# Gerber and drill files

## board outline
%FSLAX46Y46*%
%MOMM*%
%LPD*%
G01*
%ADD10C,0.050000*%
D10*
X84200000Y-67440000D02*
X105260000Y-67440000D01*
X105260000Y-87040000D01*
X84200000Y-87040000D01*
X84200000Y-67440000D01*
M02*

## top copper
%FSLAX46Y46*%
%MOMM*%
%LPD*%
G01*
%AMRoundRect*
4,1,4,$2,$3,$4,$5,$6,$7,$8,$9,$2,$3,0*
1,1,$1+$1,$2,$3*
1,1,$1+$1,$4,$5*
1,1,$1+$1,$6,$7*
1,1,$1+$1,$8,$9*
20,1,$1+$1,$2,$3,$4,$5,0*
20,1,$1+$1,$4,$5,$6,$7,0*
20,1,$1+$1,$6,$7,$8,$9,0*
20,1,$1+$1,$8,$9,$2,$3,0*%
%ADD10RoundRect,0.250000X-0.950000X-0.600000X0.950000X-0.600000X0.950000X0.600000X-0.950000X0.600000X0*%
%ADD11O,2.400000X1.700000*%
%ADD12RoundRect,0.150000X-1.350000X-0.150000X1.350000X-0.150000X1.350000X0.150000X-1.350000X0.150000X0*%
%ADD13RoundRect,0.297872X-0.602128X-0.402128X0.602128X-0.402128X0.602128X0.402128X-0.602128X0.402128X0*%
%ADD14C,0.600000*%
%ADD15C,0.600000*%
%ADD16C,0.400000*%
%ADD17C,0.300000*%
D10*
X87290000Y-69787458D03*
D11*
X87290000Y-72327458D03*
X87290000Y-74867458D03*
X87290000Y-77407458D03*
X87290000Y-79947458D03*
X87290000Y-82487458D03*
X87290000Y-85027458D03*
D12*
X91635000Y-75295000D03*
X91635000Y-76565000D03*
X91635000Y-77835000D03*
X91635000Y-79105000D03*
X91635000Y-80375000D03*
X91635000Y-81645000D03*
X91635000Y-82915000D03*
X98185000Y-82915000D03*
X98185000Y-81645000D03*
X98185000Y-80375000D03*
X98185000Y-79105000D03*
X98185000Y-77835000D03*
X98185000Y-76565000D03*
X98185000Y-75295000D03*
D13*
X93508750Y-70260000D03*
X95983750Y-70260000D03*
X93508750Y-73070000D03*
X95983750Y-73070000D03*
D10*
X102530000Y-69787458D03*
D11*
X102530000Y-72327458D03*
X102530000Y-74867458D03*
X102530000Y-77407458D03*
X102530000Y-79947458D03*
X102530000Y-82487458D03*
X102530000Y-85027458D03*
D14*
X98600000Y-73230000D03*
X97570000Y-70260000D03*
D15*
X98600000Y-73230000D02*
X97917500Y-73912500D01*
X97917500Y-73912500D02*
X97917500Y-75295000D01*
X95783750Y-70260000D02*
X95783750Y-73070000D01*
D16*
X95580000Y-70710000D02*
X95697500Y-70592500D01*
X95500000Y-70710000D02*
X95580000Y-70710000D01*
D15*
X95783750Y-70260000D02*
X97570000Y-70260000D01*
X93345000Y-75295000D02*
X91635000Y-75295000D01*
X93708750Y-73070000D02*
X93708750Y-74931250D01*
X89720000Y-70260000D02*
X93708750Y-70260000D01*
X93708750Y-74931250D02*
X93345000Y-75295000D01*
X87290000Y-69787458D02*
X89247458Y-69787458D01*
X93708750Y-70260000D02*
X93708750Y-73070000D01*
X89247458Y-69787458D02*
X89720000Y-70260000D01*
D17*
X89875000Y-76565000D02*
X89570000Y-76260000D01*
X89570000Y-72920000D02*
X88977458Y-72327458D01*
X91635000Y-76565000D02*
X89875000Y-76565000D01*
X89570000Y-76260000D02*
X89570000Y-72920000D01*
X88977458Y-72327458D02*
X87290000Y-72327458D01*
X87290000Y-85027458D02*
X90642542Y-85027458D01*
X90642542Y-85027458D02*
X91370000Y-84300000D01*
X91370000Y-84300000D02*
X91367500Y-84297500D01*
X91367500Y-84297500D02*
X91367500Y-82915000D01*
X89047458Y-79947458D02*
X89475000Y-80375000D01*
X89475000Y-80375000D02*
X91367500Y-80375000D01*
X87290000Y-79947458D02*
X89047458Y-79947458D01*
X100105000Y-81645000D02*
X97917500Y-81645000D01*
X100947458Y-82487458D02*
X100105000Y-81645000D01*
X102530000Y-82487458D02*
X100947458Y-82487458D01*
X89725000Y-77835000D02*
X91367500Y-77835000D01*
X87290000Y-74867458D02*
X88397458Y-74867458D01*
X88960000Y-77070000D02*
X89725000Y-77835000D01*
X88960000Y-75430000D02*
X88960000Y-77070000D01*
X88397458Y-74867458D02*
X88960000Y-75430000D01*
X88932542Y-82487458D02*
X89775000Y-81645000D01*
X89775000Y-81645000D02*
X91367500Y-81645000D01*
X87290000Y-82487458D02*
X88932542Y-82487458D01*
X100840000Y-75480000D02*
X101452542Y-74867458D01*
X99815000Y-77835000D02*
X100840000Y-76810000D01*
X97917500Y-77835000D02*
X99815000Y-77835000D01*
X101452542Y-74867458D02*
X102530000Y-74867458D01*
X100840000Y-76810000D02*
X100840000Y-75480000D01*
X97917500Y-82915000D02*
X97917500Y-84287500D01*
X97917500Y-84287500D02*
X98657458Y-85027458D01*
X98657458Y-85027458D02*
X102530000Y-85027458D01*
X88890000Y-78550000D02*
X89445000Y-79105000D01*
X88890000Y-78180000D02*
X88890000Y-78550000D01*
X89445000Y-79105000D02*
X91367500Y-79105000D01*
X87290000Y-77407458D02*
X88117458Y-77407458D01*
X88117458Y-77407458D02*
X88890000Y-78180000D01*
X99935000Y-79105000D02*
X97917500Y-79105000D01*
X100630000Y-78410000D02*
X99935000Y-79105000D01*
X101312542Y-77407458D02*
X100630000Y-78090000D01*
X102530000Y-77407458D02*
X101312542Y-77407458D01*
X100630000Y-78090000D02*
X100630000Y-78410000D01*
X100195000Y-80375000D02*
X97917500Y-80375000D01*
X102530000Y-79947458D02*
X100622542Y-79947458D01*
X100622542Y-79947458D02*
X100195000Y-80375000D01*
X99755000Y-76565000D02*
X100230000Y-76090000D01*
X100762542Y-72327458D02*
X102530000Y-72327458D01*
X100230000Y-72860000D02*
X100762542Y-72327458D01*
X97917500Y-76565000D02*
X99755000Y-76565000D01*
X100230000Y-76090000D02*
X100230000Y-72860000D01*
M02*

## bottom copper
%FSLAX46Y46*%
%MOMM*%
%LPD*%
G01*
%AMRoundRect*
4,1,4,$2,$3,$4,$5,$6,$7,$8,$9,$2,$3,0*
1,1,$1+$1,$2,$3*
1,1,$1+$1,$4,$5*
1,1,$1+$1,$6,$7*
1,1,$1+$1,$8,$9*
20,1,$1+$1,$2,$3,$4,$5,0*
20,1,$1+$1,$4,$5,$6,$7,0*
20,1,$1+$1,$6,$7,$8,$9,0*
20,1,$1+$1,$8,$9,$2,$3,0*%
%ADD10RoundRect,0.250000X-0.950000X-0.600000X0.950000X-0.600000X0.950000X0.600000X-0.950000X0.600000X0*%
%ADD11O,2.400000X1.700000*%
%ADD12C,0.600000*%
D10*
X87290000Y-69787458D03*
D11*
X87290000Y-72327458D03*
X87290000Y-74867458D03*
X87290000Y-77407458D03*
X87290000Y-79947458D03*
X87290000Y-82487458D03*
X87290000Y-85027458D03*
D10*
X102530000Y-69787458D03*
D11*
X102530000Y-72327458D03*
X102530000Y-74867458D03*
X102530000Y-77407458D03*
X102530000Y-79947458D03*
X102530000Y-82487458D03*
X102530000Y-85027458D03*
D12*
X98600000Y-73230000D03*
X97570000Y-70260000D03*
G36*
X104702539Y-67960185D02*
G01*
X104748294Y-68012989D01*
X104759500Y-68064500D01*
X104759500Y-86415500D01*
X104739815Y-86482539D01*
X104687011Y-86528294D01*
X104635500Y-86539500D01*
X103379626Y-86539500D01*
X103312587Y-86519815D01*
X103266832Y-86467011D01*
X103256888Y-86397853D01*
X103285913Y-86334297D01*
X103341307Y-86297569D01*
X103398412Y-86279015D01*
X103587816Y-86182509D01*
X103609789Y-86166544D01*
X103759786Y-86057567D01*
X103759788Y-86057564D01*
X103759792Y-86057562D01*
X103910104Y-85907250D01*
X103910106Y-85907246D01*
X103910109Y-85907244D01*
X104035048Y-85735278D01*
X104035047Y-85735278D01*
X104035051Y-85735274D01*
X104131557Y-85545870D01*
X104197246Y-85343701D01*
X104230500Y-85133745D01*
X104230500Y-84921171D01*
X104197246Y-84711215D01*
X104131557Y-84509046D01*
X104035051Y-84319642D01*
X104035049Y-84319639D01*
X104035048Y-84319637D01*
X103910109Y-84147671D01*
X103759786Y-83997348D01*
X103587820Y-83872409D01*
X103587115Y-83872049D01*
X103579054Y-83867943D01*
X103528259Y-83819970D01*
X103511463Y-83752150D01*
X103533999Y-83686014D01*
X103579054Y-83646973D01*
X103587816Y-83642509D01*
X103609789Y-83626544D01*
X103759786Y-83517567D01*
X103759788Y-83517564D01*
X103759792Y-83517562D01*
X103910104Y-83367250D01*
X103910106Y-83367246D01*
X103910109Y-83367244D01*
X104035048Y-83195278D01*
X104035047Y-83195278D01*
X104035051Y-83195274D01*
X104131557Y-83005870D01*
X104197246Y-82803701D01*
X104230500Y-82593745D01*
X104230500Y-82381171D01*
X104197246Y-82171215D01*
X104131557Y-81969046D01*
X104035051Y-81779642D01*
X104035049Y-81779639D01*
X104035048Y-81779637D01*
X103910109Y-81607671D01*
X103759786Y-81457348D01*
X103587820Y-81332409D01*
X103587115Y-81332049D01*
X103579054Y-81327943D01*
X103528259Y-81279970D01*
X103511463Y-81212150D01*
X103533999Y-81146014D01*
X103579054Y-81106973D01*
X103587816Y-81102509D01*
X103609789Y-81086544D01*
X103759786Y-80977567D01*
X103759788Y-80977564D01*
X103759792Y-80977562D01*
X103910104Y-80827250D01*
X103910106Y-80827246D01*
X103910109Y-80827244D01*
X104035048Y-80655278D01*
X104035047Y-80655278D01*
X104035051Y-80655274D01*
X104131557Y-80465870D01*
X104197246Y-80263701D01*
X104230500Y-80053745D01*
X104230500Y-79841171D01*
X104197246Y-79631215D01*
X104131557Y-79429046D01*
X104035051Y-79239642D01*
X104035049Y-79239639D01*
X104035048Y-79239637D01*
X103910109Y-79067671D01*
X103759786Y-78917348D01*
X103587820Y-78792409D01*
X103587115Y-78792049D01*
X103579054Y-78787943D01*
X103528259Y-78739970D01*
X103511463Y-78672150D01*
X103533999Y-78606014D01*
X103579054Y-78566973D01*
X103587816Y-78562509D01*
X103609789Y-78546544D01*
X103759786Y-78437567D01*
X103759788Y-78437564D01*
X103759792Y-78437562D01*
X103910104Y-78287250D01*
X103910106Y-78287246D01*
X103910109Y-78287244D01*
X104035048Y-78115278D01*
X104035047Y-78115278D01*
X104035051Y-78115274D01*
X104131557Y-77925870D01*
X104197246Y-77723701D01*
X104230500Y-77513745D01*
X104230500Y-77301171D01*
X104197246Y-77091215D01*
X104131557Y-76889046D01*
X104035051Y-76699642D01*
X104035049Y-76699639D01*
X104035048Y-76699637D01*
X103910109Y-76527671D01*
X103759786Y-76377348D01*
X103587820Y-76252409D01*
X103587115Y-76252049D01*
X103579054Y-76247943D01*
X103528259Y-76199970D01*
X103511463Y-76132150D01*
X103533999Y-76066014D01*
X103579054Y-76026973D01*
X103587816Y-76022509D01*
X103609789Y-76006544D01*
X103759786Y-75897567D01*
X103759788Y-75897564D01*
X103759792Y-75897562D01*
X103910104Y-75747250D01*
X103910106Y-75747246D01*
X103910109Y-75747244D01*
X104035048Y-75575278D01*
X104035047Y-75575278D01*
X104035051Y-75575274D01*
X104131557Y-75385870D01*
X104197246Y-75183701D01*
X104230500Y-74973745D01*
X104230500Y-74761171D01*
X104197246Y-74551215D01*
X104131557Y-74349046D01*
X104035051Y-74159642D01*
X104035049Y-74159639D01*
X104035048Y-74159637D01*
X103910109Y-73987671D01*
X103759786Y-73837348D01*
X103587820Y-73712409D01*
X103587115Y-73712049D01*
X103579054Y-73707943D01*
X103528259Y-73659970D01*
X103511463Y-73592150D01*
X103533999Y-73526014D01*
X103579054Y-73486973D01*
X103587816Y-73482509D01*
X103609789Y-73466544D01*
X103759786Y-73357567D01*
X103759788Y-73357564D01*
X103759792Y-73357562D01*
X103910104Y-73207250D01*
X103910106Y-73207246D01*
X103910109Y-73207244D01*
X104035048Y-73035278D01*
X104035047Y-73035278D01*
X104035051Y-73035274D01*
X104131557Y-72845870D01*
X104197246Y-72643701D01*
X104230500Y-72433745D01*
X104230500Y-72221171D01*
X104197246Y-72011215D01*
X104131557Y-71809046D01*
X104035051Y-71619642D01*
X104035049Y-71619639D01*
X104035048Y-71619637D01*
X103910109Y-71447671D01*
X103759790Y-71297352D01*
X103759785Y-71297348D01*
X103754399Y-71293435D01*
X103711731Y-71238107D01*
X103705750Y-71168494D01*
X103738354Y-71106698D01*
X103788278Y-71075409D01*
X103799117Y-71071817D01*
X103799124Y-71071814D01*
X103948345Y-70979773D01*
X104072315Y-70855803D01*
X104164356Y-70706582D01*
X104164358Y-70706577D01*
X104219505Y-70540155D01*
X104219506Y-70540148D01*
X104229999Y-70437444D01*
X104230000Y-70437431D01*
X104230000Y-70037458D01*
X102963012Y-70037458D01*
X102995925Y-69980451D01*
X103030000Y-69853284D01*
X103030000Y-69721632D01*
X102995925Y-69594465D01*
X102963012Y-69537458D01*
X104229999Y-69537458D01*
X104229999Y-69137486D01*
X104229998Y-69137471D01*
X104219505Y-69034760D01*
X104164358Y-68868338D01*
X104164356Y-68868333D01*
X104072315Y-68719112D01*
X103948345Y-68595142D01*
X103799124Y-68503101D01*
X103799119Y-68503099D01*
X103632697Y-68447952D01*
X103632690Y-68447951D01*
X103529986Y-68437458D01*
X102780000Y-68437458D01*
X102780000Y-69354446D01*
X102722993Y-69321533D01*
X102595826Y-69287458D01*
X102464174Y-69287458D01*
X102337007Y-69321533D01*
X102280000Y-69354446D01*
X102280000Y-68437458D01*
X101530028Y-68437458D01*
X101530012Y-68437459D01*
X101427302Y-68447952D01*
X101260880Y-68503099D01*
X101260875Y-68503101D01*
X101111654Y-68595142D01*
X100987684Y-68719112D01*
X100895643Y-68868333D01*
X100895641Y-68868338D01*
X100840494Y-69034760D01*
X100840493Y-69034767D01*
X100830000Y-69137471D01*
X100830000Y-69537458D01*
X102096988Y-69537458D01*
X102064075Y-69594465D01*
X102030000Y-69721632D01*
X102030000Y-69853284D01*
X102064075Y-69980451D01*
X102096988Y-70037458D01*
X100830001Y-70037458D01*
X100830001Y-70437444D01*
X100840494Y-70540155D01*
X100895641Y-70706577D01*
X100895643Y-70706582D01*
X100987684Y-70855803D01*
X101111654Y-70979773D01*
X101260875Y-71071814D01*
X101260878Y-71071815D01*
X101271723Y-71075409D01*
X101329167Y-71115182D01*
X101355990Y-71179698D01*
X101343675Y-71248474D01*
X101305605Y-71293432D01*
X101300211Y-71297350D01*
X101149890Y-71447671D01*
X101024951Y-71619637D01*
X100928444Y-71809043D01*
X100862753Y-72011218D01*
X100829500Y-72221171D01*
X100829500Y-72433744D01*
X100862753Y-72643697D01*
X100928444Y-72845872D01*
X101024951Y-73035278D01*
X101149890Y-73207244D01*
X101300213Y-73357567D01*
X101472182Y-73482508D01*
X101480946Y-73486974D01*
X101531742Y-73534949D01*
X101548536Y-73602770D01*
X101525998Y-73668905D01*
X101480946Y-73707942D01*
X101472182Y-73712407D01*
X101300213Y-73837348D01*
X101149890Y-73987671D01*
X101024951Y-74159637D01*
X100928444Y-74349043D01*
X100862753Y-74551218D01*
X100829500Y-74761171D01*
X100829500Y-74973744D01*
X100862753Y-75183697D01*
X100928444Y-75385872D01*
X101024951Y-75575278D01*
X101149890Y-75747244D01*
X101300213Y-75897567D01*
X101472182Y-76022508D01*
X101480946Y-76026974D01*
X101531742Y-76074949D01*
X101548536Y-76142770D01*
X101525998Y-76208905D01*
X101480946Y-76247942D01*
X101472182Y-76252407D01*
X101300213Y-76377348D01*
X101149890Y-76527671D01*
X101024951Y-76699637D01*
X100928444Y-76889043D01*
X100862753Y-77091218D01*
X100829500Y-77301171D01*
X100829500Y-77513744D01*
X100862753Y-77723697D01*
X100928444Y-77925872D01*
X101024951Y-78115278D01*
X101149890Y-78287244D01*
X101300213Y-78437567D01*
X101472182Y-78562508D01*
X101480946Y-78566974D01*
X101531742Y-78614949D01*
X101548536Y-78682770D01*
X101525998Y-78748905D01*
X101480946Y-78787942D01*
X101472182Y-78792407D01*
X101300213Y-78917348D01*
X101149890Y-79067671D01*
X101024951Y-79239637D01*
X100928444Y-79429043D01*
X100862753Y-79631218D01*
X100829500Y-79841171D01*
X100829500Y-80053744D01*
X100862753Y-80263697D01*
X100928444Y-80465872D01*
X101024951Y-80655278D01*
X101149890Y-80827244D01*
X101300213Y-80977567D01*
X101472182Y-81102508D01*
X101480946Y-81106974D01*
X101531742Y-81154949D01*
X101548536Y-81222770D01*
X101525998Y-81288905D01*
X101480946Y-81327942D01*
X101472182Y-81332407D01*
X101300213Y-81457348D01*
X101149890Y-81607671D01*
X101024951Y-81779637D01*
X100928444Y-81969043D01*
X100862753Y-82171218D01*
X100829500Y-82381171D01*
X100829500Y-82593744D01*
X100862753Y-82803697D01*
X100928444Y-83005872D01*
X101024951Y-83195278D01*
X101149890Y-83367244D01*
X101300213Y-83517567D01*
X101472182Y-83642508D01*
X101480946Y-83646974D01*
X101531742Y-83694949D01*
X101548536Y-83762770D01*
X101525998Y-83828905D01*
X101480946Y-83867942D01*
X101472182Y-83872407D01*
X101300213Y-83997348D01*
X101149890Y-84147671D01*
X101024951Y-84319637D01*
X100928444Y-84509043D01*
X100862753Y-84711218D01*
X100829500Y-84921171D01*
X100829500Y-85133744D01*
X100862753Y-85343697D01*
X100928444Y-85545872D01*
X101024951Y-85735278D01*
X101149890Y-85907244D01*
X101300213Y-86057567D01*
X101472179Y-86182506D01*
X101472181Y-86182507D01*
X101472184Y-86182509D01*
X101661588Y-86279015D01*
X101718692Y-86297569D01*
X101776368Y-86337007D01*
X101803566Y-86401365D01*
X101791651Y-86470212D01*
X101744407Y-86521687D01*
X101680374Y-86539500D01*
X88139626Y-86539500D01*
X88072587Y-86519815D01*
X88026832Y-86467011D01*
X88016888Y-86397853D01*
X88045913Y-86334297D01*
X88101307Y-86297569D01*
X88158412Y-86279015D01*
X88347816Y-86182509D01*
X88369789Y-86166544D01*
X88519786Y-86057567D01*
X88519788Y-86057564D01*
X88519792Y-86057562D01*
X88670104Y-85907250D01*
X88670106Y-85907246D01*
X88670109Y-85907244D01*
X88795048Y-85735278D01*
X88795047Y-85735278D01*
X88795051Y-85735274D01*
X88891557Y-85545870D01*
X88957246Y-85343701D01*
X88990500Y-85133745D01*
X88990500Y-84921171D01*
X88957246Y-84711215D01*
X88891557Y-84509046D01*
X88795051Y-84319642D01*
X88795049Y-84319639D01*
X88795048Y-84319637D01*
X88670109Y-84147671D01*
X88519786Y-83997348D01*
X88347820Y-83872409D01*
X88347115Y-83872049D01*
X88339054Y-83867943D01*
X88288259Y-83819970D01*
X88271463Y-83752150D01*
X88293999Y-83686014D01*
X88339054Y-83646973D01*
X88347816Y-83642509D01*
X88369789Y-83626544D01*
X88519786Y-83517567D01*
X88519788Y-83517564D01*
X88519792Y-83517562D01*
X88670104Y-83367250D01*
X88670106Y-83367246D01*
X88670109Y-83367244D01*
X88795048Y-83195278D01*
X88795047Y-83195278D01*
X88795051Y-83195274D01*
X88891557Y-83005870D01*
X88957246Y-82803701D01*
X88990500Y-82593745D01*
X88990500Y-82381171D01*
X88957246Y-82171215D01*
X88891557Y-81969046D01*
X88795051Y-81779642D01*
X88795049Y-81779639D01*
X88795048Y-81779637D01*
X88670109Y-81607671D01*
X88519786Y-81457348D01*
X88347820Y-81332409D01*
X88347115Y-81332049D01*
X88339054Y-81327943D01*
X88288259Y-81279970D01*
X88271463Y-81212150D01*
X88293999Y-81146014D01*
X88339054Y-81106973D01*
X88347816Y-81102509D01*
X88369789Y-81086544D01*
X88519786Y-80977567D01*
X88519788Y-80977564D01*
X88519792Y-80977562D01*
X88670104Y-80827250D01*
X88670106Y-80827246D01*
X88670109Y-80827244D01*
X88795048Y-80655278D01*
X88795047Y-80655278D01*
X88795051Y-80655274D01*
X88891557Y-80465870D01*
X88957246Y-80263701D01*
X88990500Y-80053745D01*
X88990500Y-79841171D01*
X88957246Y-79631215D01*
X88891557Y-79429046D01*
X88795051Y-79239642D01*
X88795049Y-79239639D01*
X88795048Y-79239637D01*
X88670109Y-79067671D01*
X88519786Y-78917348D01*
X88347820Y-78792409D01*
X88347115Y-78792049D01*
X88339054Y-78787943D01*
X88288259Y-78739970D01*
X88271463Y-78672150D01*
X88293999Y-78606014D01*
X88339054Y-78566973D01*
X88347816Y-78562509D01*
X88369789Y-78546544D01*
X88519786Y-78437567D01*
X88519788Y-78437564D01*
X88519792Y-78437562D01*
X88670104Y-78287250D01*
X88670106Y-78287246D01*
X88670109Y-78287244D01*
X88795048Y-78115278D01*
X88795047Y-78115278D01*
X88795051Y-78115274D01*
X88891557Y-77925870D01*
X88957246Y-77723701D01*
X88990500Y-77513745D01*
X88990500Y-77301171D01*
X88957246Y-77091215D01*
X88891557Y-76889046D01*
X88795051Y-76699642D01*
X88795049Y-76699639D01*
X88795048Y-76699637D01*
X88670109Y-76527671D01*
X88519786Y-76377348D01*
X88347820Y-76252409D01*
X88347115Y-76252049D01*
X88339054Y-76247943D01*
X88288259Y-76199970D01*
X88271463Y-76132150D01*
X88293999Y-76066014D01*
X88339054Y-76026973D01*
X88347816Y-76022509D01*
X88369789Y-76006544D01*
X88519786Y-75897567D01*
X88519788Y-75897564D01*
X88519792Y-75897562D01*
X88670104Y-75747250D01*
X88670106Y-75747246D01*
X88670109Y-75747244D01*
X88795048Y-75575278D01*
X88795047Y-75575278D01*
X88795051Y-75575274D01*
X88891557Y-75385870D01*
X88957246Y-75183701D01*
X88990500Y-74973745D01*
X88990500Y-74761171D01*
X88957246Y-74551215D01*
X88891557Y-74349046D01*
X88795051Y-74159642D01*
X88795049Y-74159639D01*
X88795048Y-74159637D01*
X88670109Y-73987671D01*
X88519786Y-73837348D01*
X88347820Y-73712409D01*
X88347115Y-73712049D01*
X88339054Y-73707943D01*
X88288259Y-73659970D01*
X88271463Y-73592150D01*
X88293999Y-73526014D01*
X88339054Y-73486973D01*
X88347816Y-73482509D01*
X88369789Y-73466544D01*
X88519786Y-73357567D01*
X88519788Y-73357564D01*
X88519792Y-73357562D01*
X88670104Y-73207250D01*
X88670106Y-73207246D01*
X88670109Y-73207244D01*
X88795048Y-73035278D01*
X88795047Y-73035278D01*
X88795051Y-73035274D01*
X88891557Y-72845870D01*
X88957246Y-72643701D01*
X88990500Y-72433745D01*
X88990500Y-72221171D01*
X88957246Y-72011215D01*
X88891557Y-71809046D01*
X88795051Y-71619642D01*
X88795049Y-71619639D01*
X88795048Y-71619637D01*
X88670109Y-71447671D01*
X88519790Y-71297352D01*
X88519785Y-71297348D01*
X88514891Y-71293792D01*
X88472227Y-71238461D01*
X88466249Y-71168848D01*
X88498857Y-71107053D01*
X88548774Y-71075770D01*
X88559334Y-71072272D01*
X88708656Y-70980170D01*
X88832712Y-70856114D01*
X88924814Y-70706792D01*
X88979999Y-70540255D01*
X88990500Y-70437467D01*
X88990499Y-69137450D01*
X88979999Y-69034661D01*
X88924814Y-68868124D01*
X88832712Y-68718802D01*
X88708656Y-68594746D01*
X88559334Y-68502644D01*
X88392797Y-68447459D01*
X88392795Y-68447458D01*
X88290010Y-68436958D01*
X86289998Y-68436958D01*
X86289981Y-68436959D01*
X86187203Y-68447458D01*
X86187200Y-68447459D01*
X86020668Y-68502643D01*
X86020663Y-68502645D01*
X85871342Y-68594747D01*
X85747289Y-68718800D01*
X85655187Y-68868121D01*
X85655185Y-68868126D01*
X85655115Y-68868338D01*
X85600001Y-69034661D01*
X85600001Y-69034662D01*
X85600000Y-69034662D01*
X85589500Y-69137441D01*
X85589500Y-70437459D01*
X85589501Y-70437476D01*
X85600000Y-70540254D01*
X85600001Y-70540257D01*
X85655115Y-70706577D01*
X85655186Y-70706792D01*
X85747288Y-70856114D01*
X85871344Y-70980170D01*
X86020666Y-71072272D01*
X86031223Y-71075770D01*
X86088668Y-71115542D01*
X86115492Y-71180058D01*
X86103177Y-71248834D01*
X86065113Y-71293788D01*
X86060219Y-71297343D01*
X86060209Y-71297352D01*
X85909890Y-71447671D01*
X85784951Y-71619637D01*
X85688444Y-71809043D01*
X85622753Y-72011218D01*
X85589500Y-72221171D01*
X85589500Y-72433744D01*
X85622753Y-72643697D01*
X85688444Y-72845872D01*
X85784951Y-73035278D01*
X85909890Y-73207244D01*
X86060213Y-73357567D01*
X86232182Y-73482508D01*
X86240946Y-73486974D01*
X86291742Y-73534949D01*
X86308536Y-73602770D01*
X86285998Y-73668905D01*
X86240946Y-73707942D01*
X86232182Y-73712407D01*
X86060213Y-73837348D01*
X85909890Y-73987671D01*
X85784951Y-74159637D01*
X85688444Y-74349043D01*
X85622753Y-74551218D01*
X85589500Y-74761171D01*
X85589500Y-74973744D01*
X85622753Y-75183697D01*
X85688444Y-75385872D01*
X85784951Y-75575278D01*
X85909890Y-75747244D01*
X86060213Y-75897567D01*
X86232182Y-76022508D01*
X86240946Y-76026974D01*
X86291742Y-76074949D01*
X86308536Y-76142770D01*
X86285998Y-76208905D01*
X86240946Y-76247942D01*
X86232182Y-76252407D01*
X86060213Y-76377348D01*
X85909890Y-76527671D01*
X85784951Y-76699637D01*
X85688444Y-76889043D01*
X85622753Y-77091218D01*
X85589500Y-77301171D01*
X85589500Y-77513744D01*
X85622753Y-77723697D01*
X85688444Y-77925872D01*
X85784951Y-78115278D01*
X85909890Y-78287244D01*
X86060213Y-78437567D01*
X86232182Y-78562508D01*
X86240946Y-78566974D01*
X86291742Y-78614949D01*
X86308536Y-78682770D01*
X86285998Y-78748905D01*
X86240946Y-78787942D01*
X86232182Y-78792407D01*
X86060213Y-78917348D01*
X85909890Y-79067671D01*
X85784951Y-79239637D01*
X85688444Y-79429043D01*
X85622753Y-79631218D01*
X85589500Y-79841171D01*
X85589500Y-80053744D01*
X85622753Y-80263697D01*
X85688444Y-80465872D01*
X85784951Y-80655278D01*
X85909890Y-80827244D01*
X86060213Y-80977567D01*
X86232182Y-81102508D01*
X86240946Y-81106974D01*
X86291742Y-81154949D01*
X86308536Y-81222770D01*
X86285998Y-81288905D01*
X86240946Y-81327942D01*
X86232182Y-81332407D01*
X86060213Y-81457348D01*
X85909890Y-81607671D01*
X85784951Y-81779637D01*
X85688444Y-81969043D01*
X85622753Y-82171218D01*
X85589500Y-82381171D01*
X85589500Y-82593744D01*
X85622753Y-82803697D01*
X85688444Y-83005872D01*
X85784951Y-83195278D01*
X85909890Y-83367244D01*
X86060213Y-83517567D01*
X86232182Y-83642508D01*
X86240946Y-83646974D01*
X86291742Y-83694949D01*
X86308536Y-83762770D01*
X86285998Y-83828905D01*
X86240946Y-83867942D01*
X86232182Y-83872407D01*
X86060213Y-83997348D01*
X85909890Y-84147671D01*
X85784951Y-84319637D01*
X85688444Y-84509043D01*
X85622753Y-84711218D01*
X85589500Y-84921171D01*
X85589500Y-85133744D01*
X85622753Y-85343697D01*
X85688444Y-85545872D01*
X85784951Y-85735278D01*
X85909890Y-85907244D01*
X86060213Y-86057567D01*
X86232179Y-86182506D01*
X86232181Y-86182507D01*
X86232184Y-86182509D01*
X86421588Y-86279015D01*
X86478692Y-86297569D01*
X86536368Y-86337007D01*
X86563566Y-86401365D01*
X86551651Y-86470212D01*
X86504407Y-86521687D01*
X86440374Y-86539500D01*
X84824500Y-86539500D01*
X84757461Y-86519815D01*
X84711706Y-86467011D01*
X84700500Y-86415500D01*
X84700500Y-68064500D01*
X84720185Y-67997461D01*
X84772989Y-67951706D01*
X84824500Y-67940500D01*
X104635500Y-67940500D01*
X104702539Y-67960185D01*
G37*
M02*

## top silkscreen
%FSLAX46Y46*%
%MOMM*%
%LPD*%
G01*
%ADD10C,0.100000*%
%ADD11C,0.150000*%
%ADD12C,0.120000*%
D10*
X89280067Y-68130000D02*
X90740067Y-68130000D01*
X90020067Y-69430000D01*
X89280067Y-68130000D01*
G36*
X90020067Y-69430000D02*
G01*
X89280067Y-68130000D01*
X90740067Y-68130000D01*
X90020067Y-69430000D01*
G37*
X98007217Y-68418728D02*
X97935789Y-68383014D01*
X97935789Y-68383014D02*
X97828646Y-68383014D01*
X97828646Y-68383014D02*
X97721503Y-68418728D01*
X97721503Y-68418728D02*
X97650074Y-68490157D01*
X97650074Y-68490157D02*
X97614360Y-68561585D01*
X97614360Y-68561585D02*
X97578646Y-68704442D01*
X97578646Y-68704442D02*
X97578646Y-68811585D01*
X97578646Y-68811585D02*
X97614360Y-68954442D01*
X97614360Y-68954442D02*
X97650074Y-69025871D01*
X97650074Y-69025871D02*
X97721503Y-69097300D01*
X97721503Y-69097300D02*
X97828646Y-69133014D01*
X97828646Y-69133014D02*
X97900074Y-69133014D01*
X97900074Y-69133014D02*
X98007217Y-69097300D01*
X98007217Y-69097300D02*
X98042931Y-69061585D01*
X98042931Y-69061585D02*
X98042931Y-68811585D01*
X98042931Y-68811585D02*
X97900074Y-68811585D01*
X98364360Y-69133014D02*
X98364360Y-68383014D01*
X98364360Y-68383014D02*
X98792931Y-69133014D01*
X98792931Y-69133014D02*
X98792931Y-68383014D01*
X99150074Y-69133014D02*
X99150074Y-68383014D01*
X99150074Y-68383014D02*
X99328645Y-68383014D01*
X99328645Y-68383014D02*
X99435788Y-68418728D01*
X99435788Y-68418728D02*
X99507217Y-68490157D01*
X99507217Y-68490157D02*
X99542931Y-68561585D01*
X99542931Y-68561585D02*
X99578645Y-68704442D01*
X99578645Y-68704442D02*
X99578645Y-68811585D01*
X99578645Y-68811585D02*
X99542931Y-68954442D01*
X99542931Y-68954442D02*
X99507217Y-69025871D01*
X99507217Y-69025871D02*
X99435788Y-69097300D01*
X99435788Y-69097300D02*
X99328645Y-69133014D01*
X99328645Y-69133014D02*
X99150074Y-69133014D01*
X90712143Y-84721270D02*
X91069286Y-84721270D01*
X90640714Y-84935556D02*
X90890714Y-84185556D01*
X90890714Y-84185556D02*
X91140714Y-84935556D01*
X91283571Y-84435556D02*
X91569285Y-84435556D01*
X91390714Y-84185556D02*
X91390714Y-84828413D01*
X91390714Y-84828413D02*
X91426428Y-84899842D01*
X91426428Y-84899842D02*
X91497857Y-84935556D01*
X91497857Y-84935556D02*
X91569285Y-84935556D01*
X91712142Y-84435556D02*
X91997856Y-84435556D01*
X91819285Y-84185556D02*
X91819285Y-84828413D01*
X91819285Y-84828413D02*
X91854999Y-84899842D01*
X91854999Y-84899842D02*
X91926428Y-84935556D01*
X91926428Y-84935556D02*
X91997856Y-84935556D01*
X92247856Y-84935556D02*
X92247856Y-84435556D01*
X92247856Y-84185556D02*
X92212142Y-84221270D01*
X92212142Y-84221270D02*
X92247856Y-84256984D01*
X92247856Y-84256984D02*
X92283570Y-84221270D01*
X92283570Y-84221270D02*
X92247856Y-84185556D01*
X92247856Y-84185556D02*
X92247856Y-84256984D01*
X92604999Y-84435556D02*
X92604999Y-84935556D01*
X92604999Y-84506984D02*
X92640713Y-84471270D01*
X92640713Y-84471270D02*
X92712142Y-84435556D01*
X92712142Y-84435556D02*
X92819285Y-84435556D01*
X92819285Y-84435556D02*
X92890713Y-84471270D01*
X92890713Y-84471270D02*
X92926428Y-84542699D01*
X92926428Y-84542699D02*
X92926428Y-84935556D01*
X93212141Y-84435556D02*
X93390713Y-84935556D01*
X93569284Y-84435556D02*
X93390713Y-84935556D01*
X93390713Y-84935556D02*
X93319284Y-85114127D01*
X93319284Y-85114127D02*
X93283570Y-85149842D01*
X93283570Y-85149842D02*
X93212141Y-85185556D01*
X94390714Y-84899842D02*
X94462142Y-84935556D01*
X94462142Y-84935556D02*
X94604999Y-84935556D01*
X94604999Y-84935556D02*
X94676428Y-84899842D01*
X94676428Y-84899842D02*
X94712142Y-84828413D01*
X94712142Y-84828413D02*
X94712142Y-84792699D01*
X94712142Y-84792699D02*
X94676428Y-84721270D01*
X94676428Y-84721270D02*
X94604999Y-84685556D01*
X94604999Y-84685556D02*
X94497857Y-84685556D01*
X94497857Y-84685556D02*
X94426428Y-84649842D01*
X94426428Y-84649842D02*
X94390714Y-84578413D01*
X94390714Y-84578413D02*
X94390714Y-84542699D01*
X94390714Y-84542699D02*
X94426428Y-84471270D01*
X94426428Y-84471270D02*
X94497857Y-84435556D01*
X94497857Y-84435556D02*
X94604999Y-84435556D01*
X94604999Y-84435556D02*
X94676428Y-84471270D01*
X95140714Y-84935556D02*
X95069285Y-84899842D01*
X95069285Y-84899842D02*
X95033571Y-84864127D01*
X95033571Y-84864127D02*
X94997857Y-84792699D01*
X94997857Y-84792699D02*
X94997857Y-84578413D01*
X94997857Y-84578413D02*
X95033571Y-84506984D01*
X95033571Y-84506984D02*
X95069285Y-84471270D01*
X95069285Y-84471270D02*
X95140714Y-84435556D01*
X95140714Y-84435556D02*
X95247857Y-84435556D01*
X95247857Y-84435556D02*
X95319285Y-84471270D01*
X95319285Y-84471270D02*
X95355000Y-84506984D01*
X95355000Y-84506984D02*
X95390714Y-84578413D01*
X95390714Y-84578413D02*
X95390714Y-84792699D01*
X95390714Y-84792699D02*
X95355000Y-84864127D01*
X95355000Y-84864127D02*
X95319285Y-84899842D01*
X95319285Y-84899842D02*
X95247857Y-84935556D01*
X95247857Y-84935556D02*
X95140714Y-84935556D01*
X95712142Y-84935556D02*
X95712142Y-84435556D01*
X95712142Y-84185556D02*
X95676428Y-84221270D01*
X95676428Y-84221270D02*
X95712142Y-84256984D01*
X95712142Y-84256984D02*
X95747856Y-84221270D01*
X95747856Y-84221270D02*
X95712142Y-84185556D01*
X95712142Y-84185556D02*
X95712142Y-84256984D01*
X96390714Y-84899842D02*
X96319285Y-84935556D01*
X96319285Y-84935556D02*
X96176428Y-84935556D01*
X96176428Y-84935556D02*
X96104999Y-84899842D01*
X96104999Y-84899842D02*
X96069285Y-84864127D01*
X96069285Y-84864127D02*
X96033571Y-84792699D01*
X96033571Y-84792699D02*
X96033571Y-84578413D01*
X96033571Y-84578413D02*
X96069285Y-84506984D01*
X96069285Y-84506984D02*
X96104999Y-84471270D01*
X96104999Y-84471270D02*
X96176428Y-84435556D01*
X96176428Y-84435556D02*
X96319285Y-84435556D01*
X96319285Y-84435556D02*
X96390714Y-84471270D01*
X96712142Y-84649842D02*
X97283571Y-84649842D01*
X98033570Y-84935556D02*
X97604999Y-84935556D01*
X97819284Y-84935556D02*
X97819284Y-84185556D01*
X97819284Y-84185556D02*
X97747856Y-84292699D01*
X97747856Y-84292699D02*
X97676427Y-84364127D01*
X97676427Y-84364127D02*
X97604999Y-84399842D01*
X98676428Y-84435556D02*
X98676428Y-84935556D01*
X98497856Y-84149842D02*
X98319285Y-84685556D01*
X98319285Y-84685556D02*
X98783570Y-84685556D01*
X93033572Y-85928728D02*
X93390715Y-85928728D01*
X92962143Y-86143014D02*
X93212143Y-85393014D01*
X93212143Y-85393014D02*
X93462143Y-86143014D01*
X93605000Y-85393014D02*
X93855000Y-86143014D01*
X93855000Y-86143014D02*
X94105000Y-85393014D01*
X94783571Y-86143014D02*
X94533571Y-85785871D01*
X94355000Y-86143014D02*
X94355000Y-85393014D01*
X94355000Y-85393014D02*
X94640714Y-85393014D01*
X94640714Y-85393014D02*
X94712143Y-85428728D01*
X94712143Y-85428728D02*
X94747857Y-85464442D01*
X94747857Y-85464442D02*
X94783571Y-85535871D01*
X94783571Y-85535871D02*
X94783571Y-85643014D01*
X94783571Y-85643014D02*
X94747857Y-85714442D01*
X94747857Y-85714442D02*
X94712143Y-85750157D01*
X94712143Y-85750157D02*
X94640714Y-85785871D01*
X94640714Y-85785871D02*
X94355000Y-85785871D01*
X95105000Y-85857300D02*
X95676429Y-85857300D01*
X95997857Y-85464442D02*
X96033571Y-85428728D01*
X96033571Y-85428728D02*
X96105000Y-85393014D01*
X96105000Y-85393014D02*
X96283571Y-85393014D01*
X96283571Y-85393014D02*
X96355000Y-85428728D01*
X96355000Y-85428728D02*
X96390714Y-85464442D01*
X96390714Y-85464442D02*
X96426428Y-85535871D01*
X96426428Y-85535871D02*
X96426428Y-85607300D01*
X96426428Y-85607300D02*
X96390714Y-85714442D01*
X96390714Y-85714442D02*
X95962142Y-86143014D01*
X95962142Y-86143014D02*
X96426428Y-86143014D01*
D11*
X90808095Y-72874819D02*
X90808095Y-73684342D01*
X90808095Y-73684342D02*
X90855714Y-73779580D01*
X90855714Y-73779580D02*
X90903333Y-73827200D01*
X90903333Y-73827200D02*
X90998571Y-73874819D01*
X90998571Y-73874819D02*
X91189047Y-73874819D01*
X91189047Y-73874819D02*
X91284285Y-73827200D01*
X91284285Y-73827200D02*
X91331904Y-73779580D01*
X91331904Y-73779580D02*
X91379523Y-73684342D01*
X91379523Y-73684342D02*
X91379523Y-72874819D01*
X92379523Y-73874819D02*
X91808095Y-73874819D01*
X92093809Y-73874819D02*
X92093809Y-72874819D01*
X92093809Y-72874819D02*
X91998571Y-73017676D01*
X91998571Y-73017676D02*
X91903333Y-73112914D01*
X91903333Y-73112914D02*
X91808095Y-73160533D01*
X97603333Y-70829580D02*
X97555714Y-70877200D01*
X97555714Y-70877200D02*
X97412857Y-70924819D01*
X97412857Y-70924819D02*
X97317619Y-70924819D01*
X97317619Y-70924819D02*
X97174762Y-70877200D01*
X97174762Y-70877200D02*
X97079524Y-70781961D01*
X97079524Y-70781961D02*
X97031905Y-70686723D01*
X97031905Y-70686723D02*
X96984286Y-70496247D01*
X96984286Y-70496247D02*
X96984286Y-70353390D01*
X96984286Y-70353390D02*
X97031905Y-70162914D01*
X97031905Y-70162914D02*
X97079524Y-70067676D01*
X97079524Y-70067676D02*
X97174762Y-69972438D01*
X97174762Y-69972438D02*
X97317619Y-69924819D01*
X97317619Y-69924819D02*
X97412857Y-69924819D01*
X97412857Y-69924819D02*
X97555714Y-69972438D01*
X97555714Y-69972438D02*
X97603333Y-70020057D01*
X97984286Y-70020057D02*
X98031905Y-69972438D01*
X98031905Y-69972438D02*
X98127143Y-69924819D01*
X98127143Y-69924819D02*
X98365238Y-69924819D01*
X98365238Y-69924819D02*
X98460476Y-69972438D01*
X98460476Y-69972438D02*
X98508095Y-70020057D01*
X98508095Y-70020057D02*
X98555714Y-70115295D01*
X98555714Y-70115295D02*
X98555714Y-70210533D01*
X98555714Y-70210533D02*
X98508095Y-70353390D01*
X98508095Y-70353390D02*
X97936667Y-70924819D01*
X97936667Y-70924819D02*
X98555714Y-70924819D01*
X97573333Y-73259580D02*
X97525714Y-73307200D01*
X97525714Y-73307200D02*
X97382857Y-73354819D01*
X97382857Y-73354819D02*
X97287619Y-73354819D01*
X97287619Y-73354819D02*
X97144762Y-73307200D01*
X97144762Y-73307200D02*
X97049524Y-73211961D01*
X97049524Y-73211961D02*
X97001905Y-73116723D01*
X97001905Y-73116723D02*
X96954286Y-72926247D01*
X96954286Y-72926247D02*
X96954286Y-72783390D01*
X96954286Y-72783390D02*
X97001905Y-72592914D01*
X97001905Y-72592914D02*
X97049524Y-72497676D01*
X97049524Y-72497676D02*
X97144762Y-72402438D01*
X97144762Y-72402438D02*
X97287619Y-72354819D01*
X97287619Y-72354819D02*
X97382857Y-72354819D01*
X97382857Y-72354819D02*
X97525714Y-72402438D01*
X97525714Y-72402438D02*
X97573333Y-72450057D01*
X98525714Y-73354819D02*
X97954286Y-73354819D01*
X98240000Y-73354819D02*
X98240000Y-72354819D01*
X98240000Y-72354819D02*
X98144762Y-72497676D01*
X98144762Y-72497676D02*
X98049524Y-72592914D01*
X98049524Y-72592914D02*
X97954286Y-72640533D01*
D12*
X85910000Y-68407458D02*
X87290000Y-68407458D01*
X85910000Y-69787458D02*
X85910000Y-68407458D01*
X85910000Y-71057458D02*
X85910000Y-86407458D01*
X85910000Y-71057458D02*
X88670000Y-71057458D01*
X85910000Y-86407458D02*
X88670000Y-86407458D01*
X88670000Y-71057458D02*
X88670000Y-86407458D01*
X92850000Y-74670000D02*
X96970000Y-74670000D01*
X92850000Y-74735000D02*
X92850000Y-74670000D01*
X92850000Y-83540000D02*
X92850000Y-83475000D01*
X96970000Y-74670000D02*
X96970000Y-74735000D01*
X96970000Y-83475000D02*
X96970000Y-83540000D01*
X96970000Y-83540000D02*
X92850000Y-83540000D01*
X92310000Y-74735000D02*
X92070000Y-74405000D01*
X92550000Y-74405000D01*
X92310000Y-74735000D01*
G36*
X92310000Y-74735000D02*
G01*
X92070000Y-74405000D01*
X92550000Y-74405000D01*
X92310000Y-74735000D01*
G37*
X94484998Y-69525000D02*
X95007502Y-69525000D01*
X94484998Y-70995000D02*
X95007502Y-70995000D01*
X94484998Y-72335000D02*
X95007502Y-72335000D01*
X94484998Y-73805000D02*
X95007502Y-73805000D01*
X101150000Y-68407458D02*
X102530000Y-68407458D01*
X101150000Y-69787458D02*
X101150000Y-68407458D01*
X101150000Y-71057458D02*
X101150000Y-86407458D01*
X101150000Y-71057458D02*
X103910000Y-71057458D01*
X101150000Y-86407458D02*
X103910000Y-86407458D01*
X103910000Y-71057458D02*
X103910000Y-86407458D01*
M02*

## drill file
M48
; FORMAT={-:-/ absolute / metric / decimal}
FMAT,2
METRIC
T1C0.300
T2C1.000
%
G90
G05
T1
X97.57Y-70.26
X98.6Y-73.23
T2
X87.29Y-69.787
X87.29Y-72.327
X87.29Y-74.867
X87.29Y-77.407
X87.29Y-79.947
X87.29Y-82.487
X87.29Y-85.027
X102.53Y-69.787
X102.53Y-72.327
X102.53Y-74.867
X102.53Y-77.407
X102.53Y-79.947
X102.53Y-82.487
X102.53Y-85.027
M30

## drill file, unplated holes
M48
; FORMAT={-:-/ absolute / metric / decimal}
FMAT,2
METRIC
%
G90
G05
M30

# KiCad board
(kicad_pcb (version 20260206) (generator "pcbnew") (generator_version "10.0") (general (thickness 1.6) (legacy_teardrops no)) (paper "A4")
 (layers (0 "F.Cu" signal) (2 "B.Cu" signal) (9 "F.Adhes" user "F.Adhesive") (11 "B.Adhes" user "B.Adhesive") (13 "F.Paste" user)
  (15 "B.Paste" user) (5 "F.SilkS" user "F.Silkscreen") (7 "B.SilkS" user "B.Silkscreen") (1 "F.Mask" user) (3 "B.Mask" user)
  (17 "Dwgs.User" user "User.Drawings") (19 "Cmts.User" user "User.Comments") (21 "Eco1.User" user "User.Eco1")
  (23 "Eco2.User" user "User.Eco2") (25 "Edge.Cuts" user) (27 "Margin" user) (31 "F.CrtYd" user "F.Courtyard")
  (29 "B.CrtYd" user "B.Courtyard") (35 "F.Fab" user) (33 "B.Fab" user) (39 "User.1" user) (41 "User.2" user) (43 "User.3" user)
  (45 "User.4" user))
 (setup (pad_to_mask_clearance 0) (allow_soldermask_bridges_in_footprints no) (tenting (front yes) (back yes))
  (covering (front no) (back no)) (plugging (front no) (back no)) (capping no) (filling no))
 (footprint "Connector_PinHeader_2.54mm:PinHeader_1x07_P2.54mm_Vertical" (layer "F.Cu") (at 87.29 69.787458)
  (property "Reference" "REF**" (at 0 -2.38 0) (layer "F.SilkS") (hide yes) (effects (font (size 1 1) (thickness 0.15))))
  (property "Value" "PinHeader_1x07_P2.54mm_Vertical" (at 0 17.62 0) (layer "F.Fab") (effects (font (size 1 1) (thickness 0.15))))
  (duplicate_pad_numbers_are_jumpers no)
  (fp_line (start -1.38 -1.38) (end 0 -1.38) (stroke (width 0.12) (type solid)) (layer "F.SilkS"))
  (fp_line (start -1.38 0) (end -1.38 -1.38) (stroke (width 0.12) (type solid)) (layer "F.SilkS"))
  (fp_line (start -1.38 1.27) (end -1.38 16.62) (stroke (width 0.12) (type solid)) (layer "F.SilkS"))
  (fp_line (start -1.38 1.27) (end 1.38 1.27) (stroke (width 0.12) (type solid)) (layer "F.SilkS"))
  (fp_line (start -1.38 16.62) (end 1.38 16.62) (stroke (width 0.12) (type solid)) (layer "F.SilkS"))
  (fp_line (start 1.38 1.27) (end 1.38 16.62) (stroke (width 0.12) (type solid)) (layer "F.SilkS"))
  (pad "1" thru_hole roundrect (at 0 0) (size 2.4 1.7) (drill 1) (layers "*.Cu" "*.Mask") (remove_unused_layers no)
   (roundrect_rratio 0.1470588235) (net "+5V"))
  (pad "2" thru_hole oval (at 0 2.54) (size 2.4 1.7) (drill 1) (layers "*.Cu" "*.Mask") (remove_unused_layers no)
   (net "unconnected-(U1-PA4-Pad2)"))
  (pad "3" thru_hole oval (at 0 5.08) (size 2.4 1.7) (drill 1) (layers "*.Cu" "*.Mask") (remove_unused_layers no)
   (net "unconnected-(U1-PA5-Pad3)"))
  (pad "4" thru_hole oval (at 0 7.62) (size 2.4 1.7) (drill 1) (layers "*.Cu" "*.Mask") (remove_unused_layers no)
   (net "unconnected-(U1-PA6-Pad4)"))
  (pad "5" thru_hole oval (at 0 10.16) (size 2.4 1.7) (drill 1) (layers "*.Cu" "*.Mask") (remove_unused_layers no)
   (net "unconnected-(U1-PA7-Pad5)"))
  (pad "6" thru_hole oval (at 0 12.7) (size 2.4 1.7) (drill 1) (layers "*.Cu" "*.Mask") (remove_unused_layers no)
   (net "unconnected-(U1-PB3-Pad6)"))
  (pad "7" thru_hole oval (at 0 15.24) (size 2.4 1.7) (drill 1) (layers "*.Cu" "*.Mask") (remove_unused_layers no)
   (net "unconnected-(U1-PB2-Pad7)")))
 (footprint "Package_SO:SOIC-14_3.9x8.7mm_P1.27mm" (layer "F.Cu") (at 94.91 79.105)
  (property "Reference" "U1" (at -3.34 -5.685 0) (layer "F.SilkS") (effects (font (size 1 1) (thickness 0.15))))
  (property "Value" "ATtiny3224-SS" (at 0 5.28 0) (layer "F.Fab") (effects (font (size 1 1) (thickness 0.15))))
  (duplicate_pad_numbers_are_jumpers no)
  (fp_line (start -2.06 -4.435) (end 2.06 -4.435) (stroke (width 0.12) (type solid)) (layer "F.SilkS"))
  (fp_line (start -2.06 -4.37) (end -2.06 -4.435) (stroke (width 0.12) (type solid)) (layer "F.SilkS"))
  (fp_line (start -2.06 4.435) (end -2.06 4.37) (stroke (width 0.12) (type solid)) (layer "F.SilkS"))
  (fp_line (start 2.06 -4.435) (end 2.06 -4.37) (stroke (width 0.12) (type solid)) (layer "F.SilkS"))
  (fp_line (start 2.06 4.37) (end 2.06 4.435) (stroke (width 0.12) (type solid)) (layer "F.SilkS"))
  (fp_line (start 2.06 4.435) (end -2.06 4.435) (stroke (width 0.12) (type solid)) (layer "F.SilkS"))
  (fp_poly (pts (xy -2.6 -4.37) (xy -2.84 -4.7) (xy -2.36 -4.7)) (stroke (width 0.12) (type solid)) (fill yes) (layer "F.SilkS"))
  (pad "1" smd roundrect (at -3.275 -3.81) (size 3 0.6) (layers "F.Cu" "F.Mask" "F.Paste") (roundrect_rratio 0.25) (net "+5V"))
  (pad "2" smd roundrect (at -3.275 -2.54) (size 3 0.6) (layers "F.Cu" "F.Mask" "F.Paste") (roundrect_rratio 0.25)
   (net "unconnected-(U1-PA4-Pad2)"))
  (pad "3" smd roundrect (at -3.275 -1.27) (size 3 0.6) (layers "F.Cu" "F.Mask" "F.Paste") (roundrect_rratio 0.25)
   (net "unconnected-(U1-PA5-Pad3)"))
  (pad "4" smd roundrect (at -3.275 0) (size 3 0.6) (layers "F.Cu" "F.Mask" "F.Paste") (roundrect_rratio 0.25)
   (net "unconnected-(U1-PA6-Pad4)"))
  (pad "5" smd roundrect (at -3.275 1.27) (size 3 0.6) (layers "F.Cu" "F.Mask" "F.Paste") (roundrect_rratio 0.25)
   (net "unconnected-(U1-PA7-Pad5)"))
  (pad "6" smd roundrect (at -3.275 2.54) (size 3 0.6) (layers "F.Cu" "F.Mask" "F.Paste") (roundrect_rratio 0.25)
   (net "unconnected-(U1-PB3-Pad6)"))
  (pad "7" smd roundrect (at -3.275 3.81) (size 3 0.6) (layers "F.Cu" "F.Mask" "F.Paste") (roundrect_rratio 0.25)
   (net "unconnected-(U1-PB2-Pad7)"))
  (pad "8" smd roundrect (at 3.275 3.81) (size 3 0.6) (layers "F.Cu" "F.Mask" "F.Paste") (roundrect_rratio 0.25)
   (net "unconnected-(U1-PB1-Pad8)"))
  (pad "9" smd roundrect (at 3.275 2.54) (size 3 0.6) (layers "F.Cu" "F.Mask" "F.Paste") (roundrect_rratio 0.25)
   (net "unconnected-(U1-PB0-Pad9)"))
  (pad "10" smd roundrect (at 3.275 1.27) (size 3 0.6) (layers "F.Cu" "F.Mask" "F.Paste") (roundrect_rratio 0.25)
   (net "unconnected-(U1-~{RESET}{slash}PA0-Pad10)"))
  (pad "11" smd roundrect (at 3.275 0) (size 3 0.6) (layers "F.Cu" "F.Mask" "F.Paste") (roundrect_rratio 0.25)
   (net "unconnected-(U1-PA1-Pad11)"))
  (pad "12" smd roundrect (at 3.275 -1.27) (size 3 0.6) (layers "F.Cu" "F.Mask" "F.Paste") (roundrect_rratio 0.25)
   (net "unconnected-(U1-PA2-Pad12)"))
  (pad "13" smd roundrect (at 3.275 -2.54) (size 3 0.6) (layers "F.Cu" "F.Mask" "F.Paste") (roundrect_rratio 0.25)
   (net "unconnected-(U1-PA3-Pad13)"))
  (pad "14" smd roundrect (at 3.275 -3.81) (size 3 0.6) (layers "F.Cu" "F.Mask" "F.Paste") (roundrect_rratio 0.25) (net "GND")))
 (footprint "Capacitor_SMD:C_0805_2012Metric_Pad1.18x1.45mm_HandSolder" (layer "F.Cu") (at 94.74625 70.26)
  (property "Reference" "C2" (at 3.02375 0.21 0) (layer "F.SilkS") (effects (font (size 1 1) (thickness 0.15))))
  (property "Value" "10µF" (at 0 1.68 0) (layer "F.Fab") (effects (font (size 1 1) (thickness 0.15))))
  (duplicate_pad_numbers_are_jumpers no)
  (fp_line (start -0.261252 -0.735) (end 0.261252 -0.735) (stroke (width 0.12) (type solid)) (layer "F.SilkS"))
  (fp_line (start -0.261252 0.735) (end 0.261252 0.735) (stroke (width 0.12) (type solid)) (layer "F.SilkS"))
  (pad "1" smd roundrect (at -1.2375 0) (size 1.8 1.4) (layers "F.Cu" "F.Mask" "F.Paste") (roundrect_rratio 0.212766) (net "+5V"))
  (pad "2" smd roundrect (at 1.2375 0) (size 1.8 1.4) (layers "F.Cu" "F.Mask" "F.Paste") (roundrect_rratio 0.212766) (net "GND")))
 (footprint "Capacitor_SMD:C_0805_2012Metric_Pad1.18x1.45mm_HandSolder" (layer "F.Cu") (at 94.74625 73.07)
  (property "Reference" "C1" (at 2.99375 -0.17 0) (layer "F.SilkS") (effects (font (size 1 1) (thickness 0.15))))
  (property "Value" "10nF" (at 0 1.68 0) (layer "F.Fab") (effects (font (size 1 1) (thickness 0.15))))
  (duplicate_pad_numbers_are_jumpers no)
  (fp_line (start -0.261252 -0.735) (end 0.261252 -0.735) (stroke (width 0.12) (type solid)) (layer "F.SilkS"))
  (fp_line (start -0.261252 0.735) (end 0.261252 0.735) (stroke (width 0.12) (type solid)) (layer "F.SilkS"))
  (pad "1" smd roundrect (at -1.2375 0) (size 1.8 1.4) (layers "F.Cu" "F.Mask" "F.Paste") (roundrect_rratio 0.212766) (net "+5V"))
  (pad "2" smd roundrect (at 1.2375 0) (size 1.8 1.4) (layers "F.Cu" "F.Mask" "F.Paste") (roundrect_rratio 0.212766) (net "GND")))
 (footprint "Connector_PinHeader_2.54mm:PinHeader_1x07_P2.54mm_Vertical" (layer "F.Cu") (at 102.53 69.787458)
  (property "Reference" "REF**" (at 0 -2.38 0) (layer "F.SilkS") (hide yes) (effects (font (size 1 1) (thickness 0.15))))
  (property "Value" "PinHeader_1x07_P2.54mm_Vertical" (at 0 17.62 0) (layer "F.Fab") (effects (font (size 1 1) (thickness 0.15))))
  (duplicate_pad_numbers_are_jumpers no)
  (fp_line (start -1.38 -1.38) (end 0 -1.38) (stroke (width 0.12) (type solid)) (layer "F.SilkS"))
  (fp_line (start -1.38 0) (end -1.38 -1.38) (stroke (width 0.12) (type solid)) (layer "F.SilkS"))
  (fp_line (start -1.38 1.27) (end -1.38 16.62) (stroke (width 0.12) (type solid)) (layer "F.SilkS"))
  (fp_line (start -1.38 1.27) (end 1.38 1.27) (stroke (width 0.12) (type solid)) (layer "F.SilkS"))
  (fp_line (start -1.38 16.62) (end 1.38 16.62) (stroke (width 0.12) (type solid)) (layer "F.SilkS"))
  (fp_line (start 1.38 1.27) (end 1.38 16.62) (stroke (width 0.12) (type solid)) (layer "F.SilkS"))
  (pad "1" thru_hole roundrect (at 0 0) (size 2.4 1.7) (drill 1) (layers "*.Cu" "*.Mask") (remove_unused_layers no)
   (roundrect_rratio 0.1470588235) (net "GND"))
  (pad "2" thru_hole oval (at 0 2.54) (size 2.4 1.7) (drill 1) (layers "*.Cu" "*.Mask") (remove_unused_layers no)
   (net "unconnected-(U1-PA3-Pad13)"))
  (pad "3" thru_hole oval (at 0 5.08) (size 2.4 1.7) (drill 1) (layers "*.Cu" "*.Mask") (remove_unused_layers no)
   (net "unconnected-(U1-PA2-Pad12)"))
  (pad "4" thru_hole oval (at 0 7.62) (size 2.4 1.7) (drill 1) (layers "*.Cu" "*.Mask") (remove_unused_layers no)
   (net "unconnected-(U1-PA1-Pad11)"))
  (pad "5" thru_hole oval (at 0 10.16) (size 2.4 1.7) (drill 1) (layers "*.Cu" "*.Mask") (remove_unused_layers no)
   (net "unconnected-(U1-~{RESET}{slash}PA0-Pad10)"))
  (pad "6" thru_hole oval (at 0 12.7) (size 2.4 1.7) (drill 1) (layers "*.Cu" "*.Mask") (remove_unused_layers no)
   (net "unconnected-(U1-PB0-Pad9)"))
  (pad "7" thru_hole oval (at 0 15.24) (size 2.4 1.7) (drill 1) (layers "*.Cu" "*.Mask") (remove_unused_layers no)
   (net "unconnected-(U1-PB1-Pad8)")))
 (gr_poly
  (pts (xy 89.280067 68.13) (xy 90.740067 68.13) (xy 90.020067 69.43)) (stroke (width 0.1) (type solid)) (fill yes) (layer "F.SilkS"))
 (gr_rect (start 84.2 67.44) (end 105.26 87.04) (stroke (width 0.05) (type default)) (fill no) (layer "Edge.Cuts"))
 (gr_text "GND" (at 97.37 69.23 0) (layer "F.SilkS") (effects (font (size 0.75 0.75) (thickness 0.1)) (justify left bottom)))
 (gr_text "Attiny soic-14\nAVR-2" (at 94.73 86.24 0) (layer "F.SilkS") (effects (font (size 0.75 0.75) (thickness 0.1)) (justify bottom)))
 (segment (start 98.6 73.23) (end 97.9175 73.9125) (width 0.6) (layer "F.Cu") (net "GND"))
 (segment (start 97.9175 73.9125) (end 97.9175 75.295) (width 0.6) (layer "F.Cu") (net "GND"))
 (segment (start 95.78375 70.26) (end 95.78375 73.07) (width 0.6) (layer "F.Cu") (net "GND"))
 (segment (start 95.58 70.71) (end 95.6975 70.5925) (width 0.4) (layer "F.Cu") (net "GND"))
 (segment (start 95.5 70.71) (end 95.58 70.71) (width 0.4) (layer "F.Cu") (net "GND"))
 (segment (start 95.78375 70.26) (end 97.57 70.26) (width 0.6) (layer "F.Cu") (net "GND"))
 (via (at 98.6 73.23) (size 0.6) (drill 0.3) (layers "F.Cu" "B.Cu") (capping no) (covering (front no) (back no))
  (plugging (front no) (back no)) (filling no) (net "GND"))
 (via (at 97.57 70.26) (size 0.6) (drill 0.3) (layers "F.Cu" "B.Cu") (capping no) (covering (front no) (back no))
  (plugging (front no) (back no)) (filling no) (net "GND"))
 (segment (start 93.345 75.295) (end 91.635 75.295) (width 0.6) (layer "F.Cu") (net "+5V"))
 (segment (start 93.70875 73.07) (end 93.70875 74.93125) (width 0.6) (layer "F.Cu") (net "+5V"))
 (segment (start 89.72 70.26) (end 93.70875 70.26) (width 0.6) (layer "F.Cu") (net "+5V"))
 (segment (start 93.70875 74.93125) (end 93.345 75.295) (width 0.6) (layer "F.Cu") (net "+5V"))
 (segment (start 87.29 69.787458) (end 89.247458 69.787458) (width 0.6) (layer "F.Cu") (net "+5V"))
 (segment (start 93.70875 70.26) (end 93.70875 73.07) (width 0.6) (layer "F.Cu") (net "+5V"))
 (segment (start 89.247458 69.787458) (end 89.72 70.26) (width 0.6) (layer "F.Cu") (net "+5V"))
 (segment (start 89.875 76.565) (end 89.57 76.26) (width 0.3) (layer "F.Cu") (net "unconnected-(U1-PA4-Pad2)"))
 (segment (start 89.57 72.92) (end 88.977458 72.327458) (width 0.3) (layer "F.Cu") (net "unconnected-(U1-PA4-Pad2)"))
 (segment (start 91.635 76.565) (end 89.875 76.565) (width 0.3) (layer "F.Cu") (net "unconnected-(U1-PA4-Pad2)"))
 (segment (start 89.57 76.26) (end 89.57 72.92) (width 0.3) (layer "F.Cu") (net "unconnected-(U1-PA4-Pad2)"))
 (segment (start 88.977458 72.327458) (end 87.29 72.327458) (width 0.3) (layer "F.Cu") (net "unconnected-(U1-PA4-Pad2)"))
 (segment (start 87.29 85.027458) (end 90.642542 85.027458) (width 0.3) (layer "F.Cu") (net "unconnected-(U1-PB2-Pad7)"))
 (segment (start 90.642542 85.027458) (end 91.37 84.3) (width 0.3) (layer "F.Cu") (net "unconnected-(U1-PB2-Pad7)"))
 (segment (start 91.37 84.3) (end 91.3675 84.2975) (width 0.3) (layer "F.Cu") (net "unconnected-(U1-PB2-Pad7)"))
 (segment (start 91.3675 84.2975) (end 91.3675 82.915) (width 0.3) (layer "F.Cu") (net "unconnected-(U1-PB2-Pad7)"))
 (segment (start 89.047458 79.947458) (end 89.475 80.375) (width 0.3) (layer "F.Cu") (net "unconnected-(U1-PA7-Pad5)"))
 (segment (start 89.475 80.375) (end 91.3675 80.375) (width 0.3) (layer "F.Cu") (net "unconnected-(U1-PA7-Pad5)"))
 (segment (start 87.29 79.947458) (end 89.047458 79.947458) (width 0.3) (layer "F.Cu") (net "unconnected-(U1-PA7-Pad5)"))
 (segment (start 100.105 81.645) (end 97.9175 81.645) (width 0.3) (layer "F.Cu") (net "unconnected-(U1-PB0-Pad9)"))
 (segment (start 100.947458 82.487458) (end 100.105 81.645) (width 0.3) (layer "F.Cu") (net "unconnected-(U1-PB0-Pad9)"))
 (segment (start 102.53 82.487458) (end 100.947458 82.487458) (width 0.3) (layer "F.Cu") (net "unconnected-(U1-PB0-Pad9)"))
 (segment (start 89.725 77.835) (end 91.3675 77.835) (width 0.3) (layer "F.Cu") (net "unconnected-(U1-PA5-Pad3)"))
 (segment (start 87.29 74.867458) (end 88.397458 74.867458) (width 0.3) (layer "F.Cu") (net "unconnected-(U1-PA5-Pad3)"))
 (segment (start 88.96 77.07) (end 89.725 77.835) (width 0.3) (layer "F.Cu") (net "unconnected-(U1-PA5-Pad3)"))
 (segment (start 88.96 75.43) (end 88.96 77.07) (width 0.3) (layer "F.Cu") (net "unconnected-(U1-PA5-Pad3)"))
 (segment (start 88.397458 74.867458) (end 88.96 75.43) (width 0.3) (layer "F.Cu") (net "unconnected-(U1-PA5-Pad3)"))
 (segment (start 88.932542 82.487458) (end 89.775 81.645) (width 0.3) (layer "F.Cu") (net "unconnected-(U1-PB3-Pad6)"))
 (segment (start 89.775 81.645) (end 91.3675 81.645) (width 0.3) (layer "F.Cu") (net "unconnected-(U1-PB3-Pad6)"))
 (segment (start 87.29 82.487458) (end 88.932542 82.487458) (width 0.3) (layer "F.Cu") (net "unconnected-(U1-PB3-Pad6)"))
 (segment (start 100.84 75.48) (end 101.452542 74.867458) (width 0.3) (layer "F.Cu") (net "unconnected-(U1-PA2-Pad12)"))
 (segment (start 99.815 77.835) (end 100.84 76.81) (width 0.3) (layer "F.Cu") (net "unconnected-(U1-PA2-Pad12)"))
 (segment (start 97.9175 77.835) (end 99.815 77.835) (width 0.3) (layer "F.Cu") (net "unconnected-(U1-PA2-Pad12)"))
 (segment (start 101.452542 74.867458) (end 102.53 74.867458) (width 0.3) (layer "F.Cu") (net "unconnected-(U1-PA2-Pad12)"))
 (segment (start 100.84 76.81) (end 100.84 75.48) (width 0.3) (layer "F.Cu") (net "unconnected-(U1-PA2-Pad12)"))
 (segment (start 97.9175 82.915) (end 97.9175 84.2875) (width 0.3) (layer "F.Cu") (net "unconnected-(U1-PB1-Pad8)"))
 (segment (start 97.9175 84.2875) (end 98.657458 85.027458) (width 0.3) (layer "F.Cu") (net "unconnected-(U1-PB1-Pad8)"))
 (segment (start 98.657458 85.027458) (end 102.53 85.027458) (width 0.3) (layer "F.Cu") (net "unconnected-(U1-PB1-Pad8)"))
 (segment (start 88.89 78.55) (end 89.445 79.105) (width 0.3) (layer "F.Cu") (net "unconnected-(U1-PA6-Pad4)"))
 (segment (start 88.89 78.18) (end 88.89 78.55) (width 0.3) (layer "F.Cu") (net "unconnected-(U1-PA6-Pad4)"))
 (segment (start 89.445 79.105) (end 91.3675 79.105) (width 0.3) (layer "F.Cu") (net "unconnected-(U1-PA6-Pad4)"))
 (segment (start 87.29 77.407458) (end 88.117458 77.407458) (width 0.3) (layer "F.Cu") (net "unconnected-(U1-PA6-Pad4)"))
 (segment (start 88.117458 77.407458) (end 88.89 78.18) (width 0.3) (layer "F.Cu") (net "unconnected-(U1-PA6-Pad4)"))
 (segment (start 99.935 79.105) (end 97.9175 79.105) (width 0.3) (layer "F.Cu") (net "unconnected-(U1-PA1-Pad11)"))
 (segment (start 100.63 78.41) (end 99.935 79.105) (width 0.3) (layer "F.Cu") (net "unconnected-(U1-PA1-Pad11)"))
 (segment (start 101.312542 77.407458) (end 100.63 78.09) (width 0.3) (layer "F.Cu") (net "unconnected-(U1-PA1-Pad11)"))
 (segment (start 102.53 77.407458) (end 101.312542 77.407458) (width 0.3) (layer "F.Cu") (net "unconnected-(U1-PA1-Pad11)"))
 (segment (start 100.63 78.09) (end 100.63 78.41) (width 0.3) (layer "F.Cu") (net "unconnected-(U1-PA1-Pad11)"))
 (segment (start 100.195 80.375) (end 97.9175 80.375) (width 0.3) (layer "F.Cu") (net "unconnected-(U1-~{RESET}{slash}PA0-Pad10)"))
 (segment (start 102.53 79.947458) (end 100.622542 79.947458) (width 0.3) (layer "F.Cu") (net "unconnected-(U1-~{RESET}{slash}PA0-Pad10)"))
 (segment (start 100.622542 79.947458) (end 100.195 80.375) (width 0.3) (layer "F.Cu") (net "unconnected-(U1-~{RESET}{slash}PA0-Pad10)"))
 (segment (start 99.755 76.565) (end 100.23 76.09) (width 0.3) (layer "F.Cu") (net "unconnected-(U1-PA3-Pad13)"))
 (segment (start 100.762542 72.327458) (end 102.53 72.327458) (width 0.3) (layer "F.Cu") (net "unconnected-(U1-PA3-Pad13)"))
 (segment (start 100.23 72.86) (end 100.762542 72.327458) (width 0.3) (layer "F.Cu") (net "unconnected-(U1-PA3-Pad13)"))
 (segment (start 97.9175 76.565) (end 99.755 76.565) (width 0.3) (layer "F.Cu") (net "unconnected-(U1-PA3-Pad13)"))
 (segment (start 100.23 76.09) (end 100.23 72.86) (width 0.3) (layer "F.Cu") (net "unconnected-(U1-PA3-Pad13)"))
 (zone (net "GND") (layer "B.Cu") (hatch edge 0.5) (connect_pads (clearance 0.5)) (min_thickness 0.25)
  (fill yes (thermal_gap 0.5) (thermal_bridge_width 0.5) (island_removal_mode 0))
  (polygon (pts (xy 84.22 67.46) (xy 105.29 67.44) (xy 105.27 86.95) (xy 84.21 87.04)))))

